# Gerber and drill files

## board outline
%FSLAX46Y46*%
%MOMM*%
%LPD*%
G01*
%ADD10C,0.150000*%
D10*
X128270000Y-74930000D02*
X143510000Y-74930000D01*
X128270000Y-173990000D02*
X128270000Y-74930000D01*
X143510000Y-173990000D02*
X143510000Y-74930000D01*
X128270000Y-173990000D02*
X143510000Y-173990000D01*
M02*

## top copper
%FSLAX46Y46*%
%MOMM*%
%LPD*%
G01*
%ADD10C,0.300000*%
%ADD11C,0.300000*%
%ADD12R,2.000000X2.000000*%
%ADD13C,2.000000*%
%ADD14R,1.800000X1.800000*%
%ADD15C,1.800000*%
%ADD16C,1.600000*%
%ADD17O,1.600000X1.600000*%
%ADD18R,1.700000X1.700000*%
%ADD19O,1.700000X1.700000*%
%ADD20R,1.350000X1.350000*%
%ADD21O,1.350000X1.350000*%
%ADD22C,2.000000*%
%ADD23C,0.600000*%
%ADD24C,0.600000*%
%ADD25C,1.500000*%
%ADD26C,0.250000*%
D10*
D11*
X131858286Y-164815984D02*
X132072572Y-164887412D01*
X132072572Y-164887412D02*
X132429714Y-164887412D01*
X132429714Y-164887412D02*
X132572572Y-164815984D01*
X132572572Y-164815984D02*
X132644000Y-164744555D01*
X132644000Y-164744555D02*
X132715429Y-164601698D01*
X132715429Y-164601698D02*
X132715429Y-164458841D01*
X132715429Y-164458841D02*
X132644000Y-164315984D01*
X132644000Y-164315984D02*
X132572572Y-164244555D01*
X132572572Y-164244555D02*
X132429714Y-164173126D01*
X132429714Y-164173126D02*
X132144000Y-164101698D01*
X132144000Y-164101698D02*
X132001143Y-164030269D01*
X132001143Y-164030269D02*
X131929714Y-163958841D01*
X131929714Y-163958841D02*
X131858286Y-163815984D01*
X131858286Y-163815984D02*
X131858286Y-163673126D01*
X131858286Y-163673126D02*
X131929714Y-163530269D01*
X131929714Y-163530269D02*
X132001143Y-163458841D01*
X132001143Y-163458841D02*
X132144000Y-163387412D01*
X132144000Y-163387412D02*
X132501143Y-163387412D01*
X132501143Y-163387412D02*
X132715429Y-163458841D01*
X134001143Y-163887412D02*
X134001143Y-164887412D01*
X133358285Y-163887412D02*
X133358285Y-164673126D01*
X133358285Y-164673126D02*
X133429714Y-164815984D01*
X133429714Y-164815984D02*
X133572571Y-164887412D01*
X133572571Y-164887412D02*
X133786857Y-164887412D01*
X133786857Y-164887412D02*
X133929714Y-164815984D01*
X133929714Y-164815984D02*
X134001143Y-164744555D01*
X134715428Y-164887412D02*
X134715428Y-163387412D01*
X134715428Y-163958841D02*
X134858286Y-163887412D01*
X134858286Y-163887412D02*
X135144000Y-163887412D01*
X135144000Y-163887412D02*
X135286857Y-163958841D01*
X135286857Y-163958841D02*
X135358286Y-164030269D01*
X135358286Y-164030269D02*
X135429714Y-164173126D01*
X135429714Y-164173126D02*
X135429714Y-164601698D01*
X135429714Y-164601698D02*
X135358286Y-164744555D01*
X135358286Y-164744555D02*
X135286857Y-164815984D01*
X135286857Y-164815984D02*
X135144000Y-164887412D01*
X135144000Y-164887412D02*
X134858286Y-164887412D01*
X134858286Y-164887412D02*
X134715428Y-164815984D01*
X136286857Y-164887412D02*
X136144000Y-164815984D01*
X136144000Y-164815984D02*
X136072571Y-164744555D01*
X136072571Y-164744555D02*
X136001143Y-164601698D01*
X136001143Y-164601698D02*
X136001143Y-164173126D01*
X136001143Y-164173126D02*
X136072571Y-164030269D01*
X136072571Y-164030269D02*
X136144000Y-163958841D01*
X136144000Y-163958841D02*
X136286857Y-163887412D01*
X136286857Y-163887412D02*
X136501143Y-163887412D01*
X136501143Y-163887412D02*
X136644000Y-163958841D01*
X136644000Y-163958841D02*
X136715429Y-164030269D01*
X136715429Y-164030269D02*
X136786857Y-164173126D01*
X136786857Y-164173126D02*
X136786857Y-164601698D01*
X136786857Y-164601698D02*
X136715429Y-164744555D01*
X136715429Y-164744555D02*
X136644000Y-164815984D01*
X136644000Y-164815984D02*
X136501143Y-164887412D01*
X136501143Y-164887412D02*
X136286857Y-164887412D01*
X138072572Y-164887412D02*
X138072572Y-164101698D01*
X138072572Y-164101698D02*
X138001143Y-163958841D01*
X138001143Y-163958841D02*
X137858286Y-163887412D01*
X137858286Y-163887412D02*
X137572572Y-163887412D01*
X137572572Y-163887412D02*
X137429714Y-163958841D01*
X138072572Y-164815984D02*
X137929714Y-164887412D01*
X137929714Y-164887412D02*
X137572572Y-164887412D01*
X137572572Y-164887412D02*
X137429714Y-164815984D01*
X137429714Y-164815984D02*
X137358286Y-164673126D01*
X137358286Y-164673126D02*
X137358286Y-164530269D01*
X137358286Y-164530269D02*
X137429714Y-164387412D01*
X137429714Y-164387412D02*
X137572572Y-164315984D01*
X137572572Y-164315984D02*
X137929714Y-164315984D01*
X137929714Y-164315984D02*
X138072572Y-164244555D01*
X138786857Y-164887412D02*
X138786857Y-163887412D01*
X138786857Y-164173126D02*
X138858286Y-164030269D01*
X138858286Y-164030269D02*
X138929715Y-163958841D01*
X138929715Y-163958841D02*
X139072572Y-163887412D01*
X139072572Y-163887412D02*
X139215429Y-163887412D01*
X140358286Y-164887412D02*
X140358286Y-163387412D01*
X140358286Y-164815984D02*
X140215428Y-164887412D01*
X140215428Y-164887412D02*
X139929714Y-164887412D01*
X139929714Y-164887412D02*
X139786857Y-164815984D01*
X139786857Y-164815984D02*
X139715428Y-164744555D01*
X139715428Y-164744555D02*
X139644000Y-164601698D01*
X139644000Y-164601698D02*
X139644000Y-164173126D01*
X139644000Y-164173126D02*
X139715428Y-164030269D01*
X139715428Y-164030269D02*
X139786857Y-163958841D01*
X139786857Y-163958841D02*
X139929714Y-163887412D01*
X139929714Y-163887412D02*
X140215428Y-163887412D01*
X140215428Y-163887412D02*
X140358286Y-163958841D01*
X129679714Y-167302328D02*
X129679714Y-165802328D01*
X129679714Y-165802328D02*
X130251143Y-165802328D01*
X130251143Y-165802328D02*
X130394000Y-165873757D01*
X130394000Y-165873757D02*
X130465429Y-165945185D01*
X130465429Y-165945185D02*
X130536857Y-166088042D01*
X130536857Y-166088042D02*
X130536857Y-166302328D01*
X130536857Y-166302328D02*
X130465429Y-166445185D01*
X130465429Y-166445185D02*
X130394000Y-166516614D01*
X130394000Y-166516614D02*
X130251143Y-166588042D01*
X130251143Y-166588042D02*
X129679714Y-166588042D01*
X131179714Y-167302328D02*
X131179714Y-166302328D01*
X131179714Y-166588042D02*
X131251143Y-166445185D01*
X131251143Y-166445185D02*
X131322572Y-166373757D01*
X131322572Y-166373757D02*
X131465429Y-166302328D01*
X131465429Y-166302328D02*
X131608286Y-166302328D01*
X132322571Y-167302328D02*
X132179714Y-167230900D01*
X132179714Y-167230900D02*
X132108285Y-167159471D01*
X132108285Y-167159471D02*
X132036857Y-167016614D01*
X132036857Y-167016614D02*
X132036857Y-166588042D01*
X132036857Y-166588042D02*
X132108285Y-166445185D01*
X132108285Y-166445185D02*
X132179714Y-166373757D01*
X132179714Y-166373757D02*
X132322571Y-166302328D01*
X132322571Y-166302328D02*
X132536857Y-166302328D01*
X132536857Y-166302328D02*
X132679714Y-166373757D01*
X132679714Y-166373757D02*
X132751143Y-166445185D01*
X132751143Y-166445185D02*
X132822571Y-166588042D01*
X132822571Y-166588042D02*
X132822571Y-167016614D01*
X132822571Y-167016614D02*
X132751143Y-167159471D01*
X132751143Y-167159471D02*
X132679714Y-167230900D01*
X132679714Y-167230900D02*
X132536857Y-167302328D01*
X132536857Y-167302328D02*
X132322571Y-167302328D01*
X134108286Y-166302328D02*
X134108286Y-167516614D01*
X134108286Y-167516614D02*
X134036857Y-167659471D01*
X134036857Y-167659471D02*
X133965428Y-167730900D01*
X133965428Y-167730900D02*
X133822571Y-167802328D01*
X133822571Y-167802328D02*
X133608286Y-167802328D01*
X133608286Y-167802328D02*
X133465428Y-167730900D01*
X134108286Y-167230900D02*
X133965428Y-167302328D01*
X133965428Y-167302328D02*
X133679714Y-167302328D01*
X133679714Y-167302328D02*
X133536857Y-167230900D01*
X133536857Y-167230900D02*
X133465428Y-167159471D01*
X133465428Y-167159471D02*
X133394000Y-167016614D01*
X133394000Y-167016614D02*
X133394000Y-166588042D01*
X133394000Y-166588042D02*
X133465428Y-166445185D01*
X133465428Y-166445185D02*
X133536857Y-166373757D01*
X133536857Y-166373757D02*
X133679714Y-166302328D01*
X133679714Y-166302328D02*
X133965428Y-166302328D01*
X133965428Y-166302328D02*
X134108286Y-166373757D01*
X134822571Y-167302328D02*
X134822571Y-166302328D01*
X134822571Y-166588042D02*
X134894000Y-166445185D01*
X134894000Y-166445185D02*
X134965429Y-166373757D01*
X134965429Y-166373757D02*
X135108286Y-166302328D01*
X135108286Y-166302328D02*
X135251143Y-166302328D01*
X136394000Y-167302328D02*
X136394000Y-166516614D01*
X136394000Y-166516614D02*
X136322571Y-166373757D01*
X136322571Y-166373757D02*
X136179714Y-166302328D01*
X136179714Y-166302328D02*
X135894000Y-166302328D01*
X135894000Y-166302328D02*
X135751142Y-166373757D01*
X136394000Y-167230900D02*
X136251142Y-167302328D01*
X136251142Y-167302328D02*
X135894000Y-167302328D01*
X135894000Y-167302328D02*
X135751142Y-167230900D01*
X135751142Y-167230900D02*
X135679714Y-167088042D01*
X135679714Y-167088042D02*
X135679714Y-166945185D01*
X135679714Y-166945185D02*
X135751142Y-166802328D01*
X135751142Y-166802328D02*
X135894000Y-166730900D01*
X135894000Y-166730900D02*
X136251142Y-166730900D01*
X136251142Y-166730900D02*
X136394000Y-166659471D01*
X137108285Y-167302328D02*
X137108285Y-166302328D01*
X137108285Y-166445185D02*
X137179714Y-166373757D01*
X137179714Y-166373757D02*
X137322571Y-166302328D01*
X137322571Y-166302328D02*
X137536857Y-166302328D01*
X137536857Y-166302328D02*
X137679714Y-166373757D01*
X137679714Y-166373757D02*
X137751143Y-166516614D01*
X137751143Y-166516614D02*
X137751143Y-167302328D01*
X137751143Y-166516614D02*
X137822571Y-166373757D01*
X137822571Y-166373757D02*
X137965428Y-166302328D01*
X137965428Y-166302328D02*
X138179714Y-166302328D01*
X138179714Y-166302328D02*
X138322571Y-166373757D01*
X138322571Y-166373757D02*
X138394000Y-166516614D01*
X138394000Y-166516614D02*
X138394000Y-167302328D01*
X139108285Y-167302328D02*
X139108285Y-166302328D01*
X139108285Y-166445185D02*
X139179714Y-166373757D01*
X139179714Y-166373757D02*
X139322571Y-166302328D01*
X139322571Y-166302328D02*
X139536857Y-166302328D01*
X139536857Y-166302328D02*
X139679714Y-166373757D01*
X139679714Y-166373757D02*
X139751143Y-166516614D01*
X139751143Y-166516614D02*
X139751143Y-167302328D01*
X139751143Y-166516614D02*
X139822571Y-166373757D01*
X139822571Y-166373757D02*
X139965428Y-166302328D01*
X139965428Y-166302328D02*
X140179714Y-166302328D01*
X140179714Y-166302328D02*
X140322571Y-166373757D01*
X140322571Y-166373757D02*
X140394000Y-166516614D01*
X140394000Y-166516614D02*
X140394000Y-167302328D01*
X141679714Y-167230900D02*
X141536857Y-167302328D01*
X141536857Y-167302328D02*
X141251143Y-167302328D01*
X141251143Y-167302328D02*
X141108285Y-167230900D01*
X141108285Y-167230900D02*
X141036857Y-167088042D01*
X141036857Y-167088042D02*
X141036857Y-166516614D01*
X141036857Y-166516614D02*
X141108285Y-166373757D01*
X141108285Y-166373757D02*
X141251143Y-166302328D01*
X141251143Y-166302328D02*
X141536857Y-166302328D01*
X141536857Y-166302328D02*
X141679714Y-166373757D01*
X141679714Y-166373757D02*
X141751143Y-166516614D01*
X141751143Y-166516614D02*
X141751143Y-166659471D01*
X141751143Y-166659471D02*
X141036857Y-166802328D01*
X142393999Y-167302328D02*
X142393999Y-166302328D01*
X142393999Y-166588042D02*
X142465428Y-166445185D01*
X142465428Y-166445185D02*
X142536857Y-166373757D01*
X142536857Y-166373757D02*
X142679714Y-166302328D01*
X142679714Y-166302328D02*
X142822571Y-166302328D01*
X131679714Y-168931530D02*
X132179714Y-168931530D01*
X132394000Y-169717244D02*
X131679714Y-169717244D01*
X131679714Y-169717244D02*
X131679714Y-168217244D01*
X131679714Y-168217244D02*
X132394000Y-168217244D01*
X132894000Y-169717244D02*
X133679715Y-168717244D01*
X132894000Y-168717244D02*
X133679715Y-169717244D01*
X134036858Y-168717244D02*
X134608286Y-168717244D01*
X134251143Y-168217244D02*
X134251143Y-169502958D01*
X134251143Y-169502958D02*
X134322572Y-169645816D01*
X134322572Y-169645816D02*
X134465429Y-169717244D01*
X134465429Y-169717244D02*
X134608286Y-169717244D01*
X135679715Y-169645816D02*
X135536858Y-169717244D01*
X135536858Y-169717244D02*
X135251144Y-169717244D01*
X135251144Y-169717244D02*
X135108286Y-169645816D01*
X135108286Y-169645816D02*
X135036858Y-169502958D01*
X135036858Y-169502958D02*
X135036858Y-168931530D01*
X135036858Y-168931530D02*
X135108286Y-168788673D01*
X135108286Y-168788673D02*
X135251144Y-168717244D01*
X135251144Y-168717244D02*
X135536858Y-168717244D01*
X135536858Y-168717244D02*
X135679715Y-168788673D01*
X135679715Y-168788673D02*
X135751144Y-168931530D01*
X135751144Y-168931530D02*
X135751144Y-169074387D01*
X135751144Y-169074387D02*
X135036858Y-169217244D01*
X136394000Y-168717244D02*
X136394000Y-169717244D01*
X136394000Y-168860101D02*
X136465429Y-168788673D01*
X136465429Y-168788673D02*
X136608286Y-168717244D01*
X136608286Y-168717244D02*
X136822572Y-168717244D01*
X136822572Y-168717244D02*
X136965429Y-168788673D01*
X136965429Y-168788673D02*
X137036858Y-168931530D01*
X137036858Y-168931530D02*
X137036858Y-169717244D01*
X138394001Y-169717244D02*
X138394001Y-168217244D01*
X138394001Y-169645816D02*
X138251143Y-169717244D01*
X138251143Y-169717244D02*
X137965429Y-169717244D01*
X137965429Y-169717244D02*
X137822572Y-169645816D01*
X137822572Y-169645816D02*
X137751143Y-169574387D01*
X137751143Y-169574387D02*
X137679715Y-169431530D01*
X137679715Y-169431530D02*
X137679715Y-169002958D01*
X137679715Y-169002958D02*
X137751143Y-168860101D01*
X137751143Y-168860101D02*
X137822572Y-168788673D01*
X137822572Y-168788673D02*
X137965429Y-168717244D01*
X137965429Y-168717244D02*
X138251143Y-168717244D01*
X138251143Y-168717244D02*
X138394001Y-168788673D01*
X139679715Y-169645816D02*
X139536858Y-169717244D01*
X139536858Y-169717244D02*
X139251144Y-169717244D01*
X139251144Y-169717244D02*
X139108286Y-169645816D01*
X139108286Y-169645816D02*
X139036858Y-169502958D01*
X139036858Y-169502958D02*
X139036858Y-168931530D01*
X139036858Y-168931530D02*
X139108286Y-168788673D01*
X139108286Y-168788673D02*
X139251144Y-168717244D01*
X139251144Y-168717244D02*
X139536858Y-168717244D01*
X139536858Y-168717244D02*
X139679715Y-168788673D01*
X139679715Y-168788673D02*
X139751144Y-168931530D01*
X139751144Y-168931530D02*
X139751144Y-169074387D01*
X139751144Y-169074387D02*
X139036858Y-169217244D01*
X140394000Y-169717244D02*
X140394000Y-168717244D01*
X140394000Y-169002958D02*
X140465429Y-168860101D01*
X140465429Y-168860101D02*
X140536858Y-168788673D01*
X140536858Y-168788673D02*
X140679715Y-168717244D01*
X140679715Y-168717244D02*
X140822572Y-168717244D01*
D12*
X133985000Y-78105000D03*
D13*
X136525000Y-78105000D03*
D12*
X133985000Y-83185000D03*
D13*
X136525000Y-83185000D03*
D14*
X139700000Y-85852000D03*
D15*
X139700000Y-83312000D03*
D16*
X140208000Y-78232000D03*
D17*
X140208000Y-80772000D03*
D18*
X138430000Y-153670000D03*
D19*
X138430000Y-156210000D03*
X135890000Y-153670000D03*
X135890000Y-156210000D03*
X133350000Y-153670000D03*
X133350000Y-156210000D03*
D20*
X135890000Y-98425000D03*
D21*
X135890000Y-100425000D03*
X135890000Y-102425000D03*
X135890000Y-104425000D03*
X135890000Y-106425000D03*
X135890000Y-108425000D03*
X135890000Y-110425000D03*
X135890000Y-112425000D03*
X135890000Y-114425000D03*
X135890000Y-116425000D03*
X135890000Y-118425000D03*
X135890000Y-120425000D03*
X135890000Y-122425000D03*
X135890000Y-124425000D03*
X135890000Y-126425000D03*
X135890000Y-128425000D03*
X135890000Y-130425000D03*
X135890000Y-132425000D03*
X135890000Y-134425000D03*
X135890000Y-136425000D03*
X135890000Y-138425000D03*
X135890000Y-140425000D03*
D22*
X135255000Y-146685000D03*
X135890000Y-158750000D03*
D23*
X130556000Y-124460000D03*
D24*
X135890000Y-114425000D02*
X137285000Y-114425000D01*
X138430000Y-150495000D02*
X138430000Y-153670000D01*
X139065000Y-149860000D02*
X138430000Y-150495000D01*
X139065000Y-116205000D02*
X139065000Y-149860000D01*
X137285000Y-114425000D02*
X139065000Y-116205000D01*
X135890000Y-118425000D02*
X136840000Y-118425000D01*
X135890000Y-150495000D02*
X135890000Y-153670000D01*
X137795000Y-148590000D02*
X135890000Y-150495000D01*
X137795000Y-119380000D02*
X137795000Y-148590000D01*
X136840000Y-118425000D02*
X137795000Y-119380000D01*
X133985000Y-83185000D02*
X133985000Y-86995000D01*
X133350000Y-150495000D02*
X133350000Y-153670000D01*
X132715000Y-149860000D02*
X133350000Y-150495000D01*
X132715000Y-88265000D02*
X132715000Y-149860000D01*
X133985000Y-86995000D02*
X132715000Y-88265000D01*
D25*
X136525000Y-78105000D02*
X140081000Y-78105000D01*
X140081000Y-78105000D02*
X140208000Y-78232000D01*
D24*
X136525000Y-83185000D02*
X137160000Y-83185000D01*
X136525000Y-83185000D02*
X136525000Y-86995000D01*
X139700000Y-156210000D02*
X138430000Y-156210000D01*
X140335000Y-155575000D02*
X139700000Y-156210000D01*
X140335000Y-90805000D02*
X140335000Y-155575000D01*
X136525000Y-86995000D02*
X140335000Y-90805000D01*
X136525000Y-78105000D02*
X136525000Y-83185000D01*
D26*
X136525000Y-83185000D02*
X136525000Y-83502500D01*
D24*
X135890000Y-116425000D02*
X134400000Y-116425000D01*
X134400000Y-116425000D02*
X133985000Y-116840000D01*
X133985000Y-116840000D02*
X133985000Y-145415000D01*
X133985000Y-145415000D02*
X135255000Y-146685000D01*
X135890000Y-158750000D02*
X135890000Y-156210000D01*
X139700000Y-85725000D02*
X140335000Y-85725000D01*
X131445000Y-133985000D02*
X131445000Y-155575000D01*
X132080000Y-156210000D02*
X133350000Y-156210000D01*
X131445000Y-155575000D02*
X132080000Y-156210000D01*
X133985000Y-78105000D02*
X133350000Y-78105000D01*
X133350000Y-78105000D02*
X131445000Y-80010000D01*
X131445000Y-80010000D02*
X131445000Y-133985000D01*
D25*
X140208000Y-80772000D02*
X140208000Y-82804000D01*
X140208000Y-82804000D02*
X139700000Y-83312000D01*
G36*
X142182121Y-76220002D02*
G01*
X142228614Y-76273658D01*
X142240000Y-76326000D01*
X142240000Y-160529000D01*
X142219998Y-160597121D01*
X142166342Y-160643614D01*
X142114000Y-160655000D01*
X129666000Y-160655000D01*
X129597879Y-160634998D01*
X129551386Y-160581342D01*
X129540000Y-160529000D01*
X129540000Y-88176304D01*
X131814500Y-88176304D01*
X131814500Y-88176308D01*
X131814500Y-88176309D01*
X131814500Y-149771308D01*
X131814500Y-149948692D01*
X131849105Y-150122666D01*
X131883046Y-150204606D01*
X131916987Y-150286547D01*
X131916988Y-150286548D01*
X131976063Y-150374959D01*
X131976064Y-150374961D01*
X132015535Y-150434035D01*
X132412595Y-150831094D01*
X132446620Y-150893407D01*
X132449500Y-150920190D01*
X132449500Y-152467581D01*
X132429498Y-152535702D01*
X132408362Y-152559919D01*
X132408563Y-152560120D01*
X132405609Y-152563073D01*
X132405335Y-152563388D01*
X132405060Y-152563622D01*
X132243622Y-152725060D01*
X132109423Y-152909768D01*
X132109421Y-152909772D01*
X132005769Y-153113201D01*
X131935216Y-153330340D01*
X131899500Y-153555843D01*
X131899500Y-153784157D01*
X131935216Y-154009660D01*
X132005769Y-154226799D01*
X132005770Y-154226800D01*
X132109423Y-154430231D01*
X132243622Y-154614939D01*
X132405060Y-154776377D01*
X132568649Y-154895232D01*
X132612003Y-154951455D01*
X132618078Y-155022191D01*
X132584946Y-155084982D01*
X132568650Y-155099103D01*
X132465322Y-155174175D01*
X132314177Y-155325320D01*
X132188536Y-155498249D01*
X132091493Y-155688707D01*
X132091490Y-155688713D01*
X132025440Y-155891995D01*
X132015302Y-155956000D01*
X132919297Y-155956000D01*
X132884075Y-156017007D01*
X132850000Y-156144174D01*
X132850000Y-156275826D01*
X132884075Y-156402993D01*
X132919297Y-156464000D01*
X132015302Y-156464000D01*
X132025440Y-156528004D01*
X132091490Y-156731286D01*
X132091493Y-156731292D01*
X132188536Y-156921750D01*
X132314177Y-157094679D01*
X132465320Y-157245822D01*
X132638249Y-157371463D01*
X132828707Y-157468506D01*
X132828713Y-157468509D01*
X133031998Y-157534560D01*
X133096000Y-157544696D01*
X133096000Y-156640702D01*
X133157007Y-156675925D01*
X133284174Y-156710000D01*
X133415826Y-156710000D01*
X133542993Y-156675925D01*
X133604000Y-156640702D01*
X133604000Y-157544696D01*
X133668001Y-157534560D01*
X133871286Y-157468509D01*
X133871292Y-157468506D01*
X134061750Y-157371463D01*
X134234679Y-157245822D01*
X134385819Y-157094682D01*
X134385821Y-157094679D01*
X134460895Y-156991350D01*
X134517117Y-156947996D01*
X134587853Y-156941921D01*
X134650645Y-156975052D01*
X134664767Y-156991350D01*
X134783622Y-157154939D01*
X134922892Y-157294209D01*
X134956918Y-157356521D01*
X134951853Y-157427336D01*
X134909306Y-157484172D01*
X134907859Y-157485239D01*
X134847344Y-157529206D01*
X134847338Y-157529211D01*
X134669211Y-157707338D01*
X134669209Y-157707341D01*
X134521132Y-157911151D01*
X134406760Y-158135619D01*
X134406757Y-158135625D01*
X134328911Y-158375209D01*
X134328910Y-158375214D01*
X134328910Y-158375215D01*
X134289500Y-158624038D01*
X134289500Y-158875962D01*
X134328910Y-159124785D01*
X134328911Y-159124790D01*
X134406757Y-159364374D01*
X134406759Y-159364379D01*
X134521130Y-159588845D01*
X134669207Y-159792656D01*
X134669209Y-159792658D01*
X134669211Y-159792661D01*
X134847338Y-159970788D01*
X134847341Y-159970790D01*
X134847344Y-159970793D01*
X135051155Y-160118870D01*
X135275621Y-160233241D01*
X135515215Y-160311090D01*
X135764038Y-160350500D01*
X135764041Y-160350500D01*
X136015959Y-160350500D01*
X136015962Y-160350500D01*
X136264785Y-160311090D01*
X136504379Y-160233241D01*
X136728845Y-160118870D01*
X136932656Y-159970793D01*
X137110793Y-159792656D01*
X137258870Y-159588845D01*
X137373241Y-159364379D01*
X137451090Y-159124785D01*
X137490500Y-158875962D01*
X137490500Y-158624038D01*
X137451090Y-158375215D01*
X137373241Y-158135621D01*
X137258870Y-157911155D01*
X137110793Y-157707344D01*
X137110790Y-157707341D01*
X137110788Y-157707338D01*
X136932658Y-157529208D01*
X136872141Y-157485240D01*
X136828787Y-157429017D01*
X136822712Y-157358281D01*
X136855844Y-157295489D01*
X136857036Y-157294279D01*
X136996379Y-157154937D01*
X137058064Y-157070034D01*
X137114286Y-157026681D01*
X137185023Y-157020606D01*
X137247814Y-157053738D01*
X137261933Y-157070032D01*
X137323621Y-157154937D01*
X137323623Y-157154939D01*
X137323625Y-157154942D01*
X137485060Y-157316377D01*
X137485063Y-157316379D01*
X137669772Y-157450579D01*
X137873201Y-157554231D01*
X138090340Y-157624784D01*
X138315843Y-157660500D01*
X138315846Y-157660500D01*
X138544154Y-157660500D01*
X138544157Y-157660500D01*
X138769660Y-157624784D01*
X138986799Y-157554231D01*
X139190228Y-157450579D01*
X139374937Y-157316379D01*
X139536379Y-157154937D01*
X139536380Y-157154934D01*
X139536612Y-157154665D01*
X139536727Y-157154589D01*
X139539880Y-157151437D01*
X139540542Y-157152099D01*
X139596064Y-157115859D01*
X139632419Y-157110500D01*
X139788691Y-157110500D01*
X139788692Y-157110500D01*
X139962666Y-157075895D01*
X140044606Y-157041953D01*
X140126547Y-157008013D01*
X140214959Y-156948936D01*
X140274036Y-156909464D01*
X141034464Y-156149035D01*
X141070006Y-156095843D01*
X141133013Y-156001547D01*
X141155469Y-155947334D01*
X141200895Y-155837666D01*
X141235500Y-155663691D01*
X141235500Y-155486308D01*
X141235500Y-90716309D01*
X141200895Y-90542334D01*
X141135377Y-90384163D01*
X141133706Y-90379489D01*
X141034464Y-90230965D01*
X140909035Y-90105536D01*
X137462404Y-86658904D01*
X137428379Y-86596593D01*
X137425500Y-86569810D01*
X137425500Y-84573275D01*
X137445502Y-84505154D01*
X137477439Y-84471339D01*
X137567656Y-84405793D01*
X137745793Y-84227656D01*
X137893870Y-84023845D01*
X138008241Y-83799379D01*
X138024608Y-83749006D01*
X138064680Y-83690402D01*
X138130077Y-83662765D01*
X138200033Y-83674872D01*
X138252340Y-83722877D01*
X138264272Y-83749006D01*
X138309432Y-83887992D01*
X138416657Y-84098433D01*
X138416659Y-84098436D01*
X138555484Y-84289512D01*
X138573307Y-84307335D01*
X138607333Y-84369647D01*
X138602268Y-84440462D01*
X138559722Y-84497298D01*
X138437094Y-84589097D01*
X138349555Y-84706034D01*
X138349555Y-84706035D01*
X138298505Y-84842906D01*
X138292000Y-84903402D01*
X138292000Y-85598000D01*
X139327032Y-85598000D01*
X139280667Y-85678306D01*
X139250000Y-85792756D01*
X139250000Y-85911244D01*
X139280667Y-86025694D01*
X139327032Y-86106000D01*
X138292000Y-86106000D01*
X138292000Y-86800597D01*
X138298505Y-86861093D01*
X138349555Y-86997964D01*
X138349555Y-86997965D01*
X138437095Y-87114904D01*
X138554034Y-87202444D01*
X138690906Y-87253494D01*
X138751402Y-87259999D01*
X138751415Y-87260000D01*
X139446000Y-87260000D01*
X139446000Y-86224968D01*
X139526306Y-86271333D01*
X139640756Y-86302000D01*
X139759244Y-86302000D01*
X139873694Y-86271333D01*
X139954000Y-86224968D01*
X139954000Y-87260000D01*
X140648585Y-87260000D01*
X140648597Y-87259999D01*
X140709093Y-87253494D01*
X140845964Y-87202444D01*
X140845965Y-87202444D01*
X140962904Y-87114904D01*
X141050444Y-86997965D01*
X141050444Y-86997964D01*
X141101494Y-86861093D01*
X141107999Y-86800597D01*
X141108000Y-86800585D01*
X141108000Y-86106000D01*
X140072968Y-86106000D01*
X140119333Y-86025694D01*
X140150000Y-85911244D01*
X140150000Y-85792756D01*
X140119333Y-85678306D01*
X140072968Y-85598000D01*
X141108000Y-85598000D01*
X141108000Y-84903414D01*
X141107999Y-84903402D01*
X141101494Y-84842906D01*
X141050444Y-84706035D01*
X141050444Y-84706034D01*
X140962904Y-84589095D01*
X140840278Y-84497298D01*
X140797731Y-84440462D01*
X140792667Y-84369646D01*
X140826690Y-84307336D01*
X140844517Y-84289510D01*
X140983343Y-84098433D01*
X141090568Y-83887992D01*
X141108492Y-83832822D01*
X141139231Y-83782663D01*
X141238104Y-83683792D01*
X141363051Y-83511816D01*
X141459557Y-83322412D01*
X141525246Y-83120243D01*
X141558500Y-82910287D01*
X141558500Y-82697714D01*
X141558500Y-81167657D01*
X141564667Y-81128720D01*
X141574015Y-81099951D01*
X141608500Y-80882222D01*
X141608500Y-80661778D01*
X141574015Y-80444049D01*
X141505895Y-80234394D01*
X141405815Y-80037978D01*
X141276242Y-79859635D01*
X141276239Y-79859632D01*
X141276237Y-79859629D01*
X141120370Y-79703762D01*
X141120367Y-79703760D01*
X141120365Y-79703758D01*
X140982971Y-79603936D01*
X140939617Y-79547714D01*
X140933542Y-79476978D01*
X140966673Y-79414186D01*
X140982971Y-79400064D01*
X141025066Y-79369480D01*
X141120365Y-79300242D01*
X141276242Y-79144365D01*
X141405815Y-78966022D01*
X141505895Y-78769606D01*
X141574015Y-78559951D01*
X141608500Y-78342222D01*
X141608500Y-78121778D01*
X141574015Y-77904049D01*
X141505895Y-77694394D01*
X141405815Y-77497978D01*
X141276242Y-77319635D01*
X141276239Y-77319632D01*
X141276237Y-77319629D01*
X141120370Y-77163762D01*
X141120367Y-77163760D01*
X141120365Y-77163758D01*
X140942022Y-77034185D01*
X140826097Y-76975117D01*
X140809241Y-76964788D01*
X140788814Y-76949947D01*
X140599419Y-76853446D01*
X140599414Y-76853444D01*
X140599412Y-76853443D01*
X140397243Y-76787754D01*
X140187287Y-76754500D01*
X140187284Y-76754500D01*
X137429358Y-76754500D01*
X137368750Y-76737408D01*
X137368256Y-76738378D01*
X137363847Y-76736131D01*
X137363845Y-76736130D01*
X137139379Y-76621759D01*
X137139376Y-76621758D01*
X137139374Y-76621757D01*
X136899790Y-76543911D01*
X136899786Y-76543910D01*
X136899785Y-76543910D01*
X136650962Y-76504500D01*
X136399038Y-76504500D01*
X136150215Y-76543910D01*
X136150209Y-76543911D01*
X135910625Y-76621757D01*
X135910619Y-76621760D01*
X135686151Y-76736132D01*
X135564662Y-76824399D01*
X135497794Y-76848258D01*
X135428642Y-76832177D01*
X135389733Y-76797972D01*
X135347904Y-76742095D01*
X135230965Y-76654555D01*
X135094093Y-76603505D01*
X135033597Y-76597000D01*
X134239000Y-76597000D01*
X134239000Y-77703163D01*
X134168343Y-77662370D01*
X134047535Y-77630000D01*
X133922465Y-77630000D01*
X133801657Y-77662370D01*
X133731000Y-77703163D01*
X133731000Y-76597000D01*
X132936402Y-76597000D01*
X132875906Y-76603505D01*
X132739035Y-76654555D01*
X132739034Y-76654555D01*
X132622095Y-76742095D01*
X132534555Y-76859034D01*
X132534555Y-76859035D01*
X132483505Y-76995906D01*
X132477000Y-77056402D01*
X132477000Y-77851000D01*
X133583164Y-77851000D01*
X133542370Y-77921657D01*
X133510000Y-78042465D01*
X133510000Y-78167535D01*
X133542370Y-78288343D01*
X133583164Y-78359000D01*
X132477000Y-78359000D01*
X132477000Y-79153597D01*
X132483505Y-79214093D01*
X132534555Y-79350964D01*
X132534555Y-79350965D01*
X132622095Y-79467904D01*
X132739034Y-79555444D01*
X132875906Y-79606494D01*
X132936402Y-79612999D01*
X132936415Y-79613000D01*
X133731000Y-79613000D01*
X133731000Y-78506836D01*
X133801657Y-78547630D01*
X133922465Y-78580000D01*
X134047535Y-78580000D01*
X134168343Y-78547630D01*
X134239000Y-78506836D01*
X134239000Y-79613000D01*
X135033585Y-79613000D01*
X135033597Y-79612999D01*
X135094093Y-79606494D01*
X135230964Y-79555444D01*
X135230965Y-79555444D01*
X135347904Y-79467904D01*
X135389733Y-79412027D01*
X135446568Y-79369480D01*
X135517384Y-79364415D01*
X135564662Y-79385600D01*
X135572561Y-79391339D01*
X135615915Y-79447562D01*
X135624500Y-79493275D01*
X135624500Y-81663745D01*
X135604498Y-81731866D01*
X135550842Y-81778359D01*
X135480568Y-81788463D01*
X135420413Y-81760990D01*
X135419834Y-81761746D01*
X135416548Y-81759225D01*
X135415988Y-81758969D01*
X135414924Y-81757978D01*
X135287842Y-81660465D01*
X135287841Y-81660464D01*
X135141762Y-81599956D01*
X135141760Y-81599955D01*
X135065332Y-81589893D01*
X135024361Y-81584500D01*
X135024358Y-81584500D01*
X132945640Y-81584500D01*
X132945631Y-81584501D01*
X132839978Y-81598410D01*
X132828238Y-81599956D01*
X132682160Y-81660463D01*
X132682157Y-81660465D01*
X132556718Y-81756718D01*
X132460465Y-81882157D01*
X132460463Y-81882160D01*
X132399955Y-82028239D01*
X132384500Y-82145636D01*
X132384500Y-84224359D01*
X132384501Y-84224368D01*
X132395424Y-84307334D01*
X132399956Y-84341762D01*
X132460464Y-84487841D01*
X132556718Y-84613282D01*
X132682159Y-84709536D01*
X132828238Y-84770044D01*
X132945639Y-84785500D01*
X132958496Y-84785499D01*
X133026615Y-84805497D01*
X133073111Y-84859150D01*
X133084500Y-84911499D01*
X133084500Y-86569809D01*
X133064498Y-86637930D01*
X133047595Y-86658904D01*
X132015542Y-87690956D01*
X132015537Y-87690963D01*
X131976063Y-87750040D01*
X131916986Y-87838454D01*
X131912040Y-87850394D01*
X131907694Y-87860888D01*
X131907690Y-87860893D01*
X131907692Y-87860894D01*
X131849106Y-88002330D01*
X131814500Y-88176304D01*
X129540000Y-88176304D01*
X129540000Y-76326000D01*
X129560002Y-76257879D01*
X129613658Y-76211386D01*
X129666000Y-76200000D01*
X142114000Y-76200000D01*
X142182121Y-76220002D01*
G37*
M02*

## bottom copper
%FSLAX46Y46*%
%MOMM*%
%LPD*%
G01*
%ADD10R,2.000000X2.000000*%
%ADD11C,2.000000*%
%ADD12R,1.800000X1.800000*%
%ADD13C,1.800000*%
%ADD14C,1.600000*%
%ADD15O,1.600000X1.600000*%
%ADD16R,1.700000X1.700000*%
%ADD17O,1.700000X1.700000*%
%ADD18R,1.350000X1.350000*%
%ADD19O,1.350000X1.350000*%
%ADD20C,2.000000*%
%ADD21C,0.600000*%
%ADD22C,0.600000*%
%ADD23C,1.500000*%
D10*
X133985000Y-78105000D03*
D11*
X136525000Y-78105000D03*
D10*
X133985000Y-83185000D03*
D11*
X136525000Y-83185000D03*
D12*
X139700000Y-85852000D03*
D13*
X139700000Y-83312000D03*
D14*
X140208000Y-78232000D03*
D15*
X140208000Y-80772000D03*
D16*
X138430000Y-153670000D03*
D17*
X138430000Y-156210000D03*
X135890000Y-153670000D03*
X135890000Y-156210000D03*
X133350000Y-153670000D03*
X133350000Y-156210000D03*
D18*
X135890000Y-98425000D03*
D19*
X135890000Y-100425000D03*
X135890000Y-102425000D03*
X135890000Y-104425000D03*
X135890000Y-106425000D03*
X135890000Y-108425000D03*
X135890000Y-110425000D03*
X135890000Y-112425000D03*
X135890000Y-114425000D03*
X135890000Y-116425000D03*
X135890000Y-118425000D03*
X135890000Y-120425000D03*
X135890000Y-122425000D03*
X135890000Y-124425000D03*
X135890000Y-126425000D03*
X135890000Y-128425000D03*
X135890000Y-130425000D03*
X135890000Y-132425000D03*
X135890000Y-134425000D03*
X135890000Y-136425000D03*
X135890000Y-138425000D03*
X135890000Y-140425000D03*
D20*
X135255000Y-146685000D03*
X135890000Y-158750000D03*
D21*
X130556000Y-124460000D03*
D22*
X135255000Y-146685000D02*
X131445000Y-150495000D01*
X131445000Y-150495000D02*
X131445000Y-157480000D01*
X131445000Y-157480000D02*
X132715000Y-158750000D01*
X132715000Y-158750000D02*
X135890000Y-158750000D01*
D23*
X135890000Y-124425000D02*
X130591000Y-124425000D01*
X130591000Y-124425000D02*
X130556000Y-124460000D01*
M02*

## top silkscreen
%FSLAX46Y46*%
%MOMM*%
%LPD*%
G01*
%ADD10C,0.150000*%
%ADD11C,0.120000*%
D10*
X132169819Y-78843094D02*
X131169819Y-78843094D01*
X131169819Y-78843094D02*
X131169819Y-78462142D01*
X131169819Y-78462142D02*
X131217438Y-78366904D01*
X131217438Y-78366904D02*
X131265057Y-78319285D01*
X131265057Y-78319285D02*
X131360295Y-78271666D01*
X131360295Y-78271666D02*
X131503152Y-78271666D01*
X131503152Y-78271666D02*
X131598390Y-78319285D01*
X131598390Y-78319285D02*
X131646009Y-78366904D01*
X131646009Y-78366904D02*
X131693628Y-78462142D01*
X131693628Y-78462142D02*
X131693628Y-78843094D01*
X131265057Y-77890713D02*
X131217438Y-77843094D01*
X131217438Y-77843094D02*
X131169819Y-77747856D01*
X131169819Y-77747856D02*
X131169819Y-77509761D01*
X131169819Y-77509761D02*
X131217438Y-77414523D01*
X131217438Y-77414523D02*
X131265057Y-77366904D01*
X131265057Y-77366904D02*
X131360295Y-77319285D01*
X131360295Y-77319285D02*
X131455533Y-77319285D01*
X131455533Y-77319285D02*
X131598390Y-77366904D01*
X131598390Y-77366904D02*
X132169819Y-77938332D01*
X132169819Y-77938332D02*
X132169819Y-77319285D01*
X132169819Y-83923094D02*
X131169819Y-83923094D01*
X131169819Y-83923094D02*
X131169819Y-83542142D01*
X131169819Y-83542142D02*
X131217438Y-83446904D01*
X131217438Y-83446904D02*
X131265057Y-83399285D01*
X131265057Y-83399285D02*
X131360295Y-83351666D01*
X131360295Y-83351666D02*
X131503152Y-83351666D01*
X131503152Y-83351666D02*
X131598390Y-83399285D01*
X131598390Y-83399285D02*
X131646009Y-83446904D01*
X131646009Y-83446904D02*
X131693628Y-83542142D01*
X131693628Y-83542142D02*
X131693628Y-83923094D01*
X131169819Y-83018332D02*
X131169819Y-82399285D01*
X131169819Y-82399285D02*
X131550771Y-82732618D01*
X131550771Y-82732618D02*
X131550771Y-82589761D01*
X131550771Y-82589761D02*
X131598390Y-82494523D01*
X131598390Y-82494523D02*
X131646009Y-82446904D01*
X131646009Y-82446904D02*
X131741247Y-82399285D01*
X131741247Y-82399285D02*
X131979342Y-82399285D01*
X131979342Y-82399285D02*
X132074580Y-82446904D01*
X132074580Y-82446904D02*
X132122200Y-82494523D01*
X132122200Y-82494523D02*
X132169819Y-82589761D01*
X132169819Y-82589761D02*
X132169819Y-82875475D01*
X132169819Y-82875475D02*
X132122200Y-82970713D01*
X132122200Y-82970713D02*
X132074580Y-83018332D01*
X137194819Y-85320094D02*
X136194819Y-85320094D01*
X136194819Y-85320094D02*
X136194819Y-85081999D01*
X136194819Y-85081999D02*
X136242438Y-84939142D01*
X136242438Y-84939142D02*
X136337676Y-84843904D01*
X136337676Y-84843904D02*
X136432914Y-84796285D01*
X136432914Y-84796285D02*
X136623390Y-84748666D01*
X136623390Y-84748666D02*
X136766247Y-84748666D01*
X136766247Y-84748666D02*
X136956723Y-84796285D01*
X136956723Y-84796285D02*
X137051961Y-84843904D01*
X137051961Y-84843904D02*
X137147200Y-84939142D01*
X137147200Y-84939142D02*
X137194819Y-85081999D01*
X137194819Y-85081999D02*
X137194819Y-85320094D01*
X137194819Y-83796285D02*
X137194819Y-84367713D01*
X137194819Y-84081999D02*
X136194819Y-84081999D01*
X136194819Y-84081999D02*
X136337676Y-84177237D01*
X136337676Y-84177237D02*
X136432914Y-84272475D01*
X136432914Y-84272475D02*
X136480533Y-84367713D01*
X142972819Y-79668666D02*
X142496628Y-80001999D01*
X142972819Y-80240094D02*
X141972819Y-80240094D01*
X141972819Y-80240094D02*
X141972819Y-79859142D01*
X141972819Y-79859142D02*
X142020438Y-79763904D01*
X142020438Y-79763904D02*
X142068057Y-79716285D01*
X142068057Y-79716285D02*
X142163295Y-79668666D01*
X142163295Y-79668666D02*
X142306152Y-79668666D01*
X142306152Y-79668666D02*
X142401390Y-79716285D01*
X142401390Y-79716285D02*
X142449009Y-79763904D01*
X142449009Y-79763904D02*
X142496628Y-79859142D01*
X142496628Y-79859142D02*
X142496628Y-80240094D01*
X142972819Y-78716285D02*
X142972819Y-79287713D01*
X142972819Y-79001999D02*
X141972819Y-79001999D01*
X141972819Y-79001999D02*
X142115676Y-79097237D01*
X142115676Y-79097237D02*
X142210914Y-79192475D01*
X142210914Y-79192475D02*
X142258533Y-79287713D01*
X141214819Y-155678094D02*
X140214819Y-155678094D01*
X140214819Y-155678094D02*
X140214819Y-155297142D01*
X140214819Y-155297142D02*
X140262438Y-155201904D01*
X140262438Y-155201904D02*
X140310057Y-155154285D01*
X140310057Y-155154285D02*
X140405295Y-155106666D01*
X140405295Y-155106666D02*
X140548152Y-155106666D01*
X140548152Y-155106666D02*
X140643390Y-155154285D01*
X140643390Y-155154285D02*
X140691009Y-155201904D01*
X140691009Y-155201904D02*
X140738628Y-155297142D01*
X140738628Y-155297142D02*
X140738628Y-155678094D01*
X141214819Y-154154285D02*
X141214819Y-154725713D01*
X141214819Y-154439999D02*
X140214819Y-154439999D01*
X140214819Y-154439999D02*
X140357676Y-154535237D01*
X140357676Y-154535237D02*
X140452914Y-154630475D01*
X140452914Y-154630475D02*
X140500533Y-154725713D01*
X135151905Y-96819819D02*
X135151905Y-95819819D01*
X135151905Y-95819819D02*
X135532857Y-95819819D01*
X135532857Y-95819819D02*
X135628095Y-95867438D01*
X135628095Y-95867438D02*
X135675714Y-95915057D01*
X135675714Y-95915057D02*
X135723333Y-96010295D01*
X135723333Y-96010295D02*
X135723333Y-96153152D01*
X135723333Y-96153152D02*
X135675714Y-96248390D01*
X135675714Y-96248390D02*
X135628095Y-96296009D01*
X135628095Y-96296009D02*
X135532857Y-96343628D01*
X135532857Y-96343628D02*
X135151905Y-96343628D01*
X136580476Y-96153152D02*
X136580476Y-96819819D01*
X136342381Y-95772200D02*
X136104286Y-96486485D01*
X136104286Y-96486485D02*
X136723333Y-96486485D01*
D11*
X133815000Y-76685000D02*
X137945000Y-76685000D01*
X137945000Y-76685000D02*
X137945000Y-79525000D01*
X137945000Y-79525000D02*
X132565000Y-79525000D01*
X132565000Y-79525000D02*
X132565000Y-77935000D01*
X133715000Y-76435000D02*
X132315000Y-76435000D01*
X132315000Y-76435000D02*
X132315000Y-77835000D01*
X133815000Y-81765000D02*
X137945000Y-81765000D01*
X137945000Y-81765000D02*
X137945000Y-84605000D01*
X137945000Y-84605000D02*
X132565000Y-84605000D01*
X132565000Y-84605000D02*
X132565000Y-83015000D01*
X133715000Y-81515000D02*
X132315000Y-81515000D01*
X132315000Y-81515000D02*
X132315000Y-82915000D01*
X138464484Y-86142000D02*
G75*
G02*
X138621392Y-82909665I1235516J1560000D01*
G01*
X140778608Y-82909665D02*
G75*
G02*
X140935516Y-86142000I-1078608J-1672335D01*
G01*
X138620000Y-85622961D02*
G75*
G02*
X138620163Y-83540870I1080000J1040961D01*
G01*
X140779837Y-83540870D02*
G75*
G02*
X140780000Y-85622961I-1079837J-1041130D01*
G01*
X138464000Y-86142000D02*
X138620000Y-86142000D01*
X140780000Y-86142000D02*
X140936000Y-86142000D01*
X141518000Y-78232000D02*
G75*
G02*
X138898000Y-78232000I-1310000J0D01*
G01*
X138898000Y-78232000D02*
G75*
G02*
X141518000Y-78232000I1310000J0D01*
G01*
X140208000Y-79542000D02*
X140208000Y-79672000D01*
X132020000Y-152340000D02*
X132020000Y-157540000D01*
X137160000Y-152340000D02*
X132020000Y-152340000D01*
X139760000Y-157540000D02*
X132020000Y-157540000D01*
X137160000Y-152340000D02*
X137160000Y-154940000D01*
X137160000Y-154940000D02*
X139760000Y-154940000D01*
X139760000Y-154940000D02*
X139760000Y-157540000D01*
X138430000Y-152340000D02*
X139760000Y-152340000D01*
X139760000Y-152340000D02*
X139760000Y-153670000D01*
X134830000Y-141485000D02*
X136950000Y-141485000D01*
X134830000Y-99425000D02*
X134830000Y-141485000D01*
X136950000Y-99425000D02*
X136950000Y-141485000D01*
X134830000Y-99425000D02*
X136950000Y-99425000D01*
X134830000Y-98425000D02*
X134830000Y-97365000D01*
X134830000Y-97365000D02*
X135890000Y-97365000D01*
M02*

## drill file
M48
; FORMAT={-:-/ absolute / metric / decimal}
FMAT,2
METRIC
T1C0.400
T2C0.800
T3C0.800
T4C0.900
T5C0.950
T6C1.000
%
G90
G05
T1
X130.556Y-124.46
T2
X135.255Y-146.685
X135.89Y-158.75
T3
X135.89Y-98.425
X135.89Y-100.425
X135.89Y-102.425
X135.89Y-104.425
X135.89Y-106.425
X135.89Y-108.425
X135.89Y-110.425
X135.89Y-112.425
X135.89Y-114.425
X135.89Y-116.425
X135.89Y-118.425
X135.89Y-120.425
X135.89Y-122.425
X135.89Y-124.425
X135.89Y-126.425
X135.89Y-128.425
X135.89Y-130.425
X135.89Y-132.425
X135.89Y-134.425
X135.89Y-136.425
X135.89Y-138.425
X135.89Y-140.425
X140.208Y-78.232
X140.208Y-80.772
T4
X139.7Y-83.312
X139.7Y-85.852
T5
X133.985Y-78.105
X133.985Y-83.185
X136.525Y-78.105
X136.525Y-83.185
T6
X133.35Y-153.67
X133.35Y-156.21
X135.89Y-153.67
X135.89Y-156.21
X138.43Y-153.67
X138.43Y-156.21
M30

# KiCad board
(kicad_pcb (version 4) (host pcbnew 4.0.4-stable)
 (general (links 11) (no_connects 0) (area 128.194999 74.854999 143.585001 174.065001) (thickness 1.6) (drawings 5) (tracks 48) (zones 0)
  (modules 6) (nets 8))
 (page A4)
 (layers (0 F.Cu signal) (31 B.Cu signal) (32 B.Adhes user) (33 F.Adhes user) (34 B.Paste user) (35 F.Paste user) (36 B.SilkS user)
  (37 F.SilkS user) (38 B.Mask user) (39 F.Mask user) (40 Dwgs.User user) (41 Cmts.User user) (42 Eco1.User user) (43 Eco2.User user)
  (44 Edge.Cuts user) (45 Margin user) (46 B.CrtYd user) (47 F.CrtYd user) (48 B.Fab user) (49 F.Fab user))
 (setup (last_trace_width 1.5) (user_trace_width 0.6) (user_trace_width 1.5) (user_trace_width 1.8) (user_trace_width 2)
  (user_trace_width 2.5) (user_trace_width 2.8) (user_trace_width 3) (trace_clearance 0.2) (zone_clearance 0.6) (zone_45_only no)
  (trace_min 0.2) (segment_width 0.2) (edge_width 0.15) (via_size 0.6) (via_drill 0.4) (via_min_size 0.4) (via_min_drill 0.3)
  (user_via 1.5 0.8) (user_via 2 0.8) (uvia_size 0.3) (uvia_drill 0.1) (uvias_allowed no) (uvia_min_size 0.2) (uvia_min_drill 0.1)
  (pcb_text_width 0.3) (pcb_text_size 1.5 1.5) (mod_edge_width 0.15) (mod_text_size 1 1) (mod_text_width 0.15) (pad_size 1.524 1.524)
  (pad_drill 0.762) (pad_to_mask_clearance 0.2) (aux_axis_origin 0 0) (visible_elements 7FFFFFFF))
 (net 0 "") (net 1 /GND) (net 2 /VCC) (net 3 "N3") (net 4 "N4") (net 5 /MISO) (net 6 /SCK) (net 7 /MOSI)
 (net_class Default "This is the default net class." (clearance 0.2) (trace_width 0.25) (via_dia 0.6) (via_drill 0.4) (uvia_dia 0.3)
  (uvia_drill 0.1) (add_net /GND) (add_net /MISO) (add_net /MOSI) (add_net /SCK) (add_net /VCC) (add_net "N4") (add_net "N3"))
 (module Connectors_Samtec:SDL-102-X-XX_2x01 (layer F.Cu) (at 133.985 78.105)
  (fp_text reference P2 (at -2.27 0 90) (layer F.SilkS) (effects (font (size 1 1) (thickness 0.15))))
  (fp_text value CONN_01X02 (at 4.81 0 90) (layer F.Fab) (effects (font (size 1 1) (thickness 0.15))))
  (fp_line (start -0.17 -1.42) (end 3.96 -1.42) (layer F.SilkS) (width 0.12))
  (fp_line (start 3.96 -1.42) (end 3.96 1.42) (layer F.SilkS) (width 0.12))
  (fp_line (start 3.96 1.42) (end -1.42 1.42) (layer F.SilkS) (width 0.12))
  (fp_line (start -1.42 1.42) (end -1.42 -0.17) (layer F.SilkS) (width 0.12))
  (fp_line (start -0.27 -1.67) (end -1.67 -1.67) (layer F.SilkS) (width 0.12))
  (fp_line (start -1.67 -1.67) (end -1.67 -0.27) (layer F.SilkS) (width 0.12))
  (pad 1 thru_hole rect (at 0 0) (size 2 2) (drill 0.95) (layers *.Cu *.Mask) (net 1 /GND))
  (pad 2 thru_hole circle (at 2.54 0) (size 2 2) (drill 0.95) (layers *.Cu *.Mask) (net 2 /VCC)))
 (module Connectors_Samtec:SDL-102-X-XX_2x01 (layer F.Cu) (at 133.985 83.185)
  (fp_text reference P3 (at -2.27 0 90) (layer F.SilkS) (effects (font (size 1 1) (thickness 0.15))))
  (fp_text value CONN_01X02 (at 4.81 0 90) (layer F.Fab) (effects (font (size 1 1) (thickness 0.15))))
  (fp_line (start -0.17 -1.42) (end 3.96 -1.42) (layer F.SilkS) (width 0.12))
  (fp_line (start 3.96 -1.42) (end 3.96 1.42) (layer F.SilkS) (width 0.12))
  (fp_line (start 3.96 1.42) (end -1.42 1.42) (layer F.SilkS) (width 0.12))
  (fp_line (start -1.42 1.42) (end -1.42 -0.17) (layer F.SilkS) (width 0.12))
  (fp_line (start -0.27 -1.67) (end -1.67 -1.67) (layer F.SilkS) (width 0.12))
  (fp_line (start -1.67 -1.67) (end -1.67 -0.27) (layer F.SilkS) (width 0.12))
  (pad 1 thru_hole rect (at 0 0) (size 2 2) (drill 0.95) (layers *.Cu *.Mask) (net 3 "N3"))
  (pad 2 thru_hole circle (at 2.54 0) (size 2 2) (drill 0.95) (layers *.Cu *.Mask) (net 2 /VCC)))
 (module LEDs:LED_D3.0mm (layer F.Cu) (at 139.7 85.852 90)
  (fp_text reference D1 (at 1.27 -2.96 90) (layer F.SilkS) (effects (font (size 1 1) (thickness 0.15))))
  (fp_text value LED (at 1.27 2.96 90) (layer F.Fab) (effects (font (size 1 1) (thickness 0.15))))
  (fp_arc (start 1.27 0) (end -0.29 -1.235516) (angle 108.8) (layer F.SilkS) (width 0.12))
  (fp_arc (start 1.27 0) (end -0.29 1.235516) (angle -108.8) (layer F.SilkS) (width 0.12))
  (fp_arc (start 1.27 0) (end 0.229039 -1.08) (angle 87.9) (layer F.SilkS) (width 0.12))
  (fp_arc (start 1.27 0) (end 0.229039 1.08) (angle -87.9) (layer F.SilkS) (width 0.12))
  (fp_line (start -0.29 -1.236) (end -0.29 -1.08) (layer F.SilkS) (width 0.12))
  (fp_line (start -0.29 1.08) (end -0.29 1.236) (layer F.SilkS) (width 0.12))
  (pad 1 thru_hole rect (at 0 0 90) (size 1.8 1.8) (drill 0.9) (layers *.Cu *.Mask) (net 1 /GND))
  (pad 2 thru_hole circle (at 2.54 0 90) (size 1.8 1.8) (drill 0.9) (layers *.Cu *.Mask) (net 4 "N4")))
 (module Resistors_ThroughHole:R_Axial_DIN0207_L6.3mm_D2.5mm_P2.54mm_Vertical (layer F.Cu) (at 140.208 78.232 270)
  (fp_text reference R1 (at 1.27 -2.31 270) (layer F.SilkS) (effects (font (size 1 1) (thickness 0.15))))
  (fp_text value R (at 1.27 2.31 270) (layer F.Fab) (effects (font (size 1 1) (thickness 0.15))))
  (fp_circle (center 0 0) (end 1.31 0) (layer F.SilkS) (width 0.12))
  (fp_line (start 1.31 0) (end 1.44 0) (layer F.SilkS) (width 0.12))
  (pad 1 thru_hole circle (at 0 0 270) (size 1.6 1.6) (drill 0.8) (layers *.Cu *.Mask) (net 2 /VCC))
  (pad 2 thru_hole oval (at 2.54 0 270) (size 1.6 1.6) (drill 0.8) (layers *.Cu *.Mask) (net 4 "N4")))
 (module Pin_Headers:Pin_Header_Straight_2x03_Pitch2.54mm (layer F.Cu) (at 138.43 153.67 270)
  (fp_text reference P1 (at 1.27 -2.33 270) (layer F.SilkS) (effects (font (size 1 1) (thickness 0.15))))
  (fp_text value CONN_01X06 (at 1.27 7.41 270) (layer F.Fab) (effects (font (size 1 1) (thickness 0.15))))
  (fp_line (start -1.33 6.41) (end 3.87 6.41) (layer F.SilkS) (width 0.12))
  (fp_line (start -1.33 1.27) (end -1.33 6.41) (layer F.SilkS) (width 0.12))
  (fp_line (start 3.87 -1.33) (end 3.87 6.41) (layer F.SilkS) (width 0.12))
  (fp_line (start -1.33 1.27) (end 1.27 1.27) (layer F.SilkS) (width 0.12))
  (fp_line (start 1.27 1.27) (end 1.27 -1.33) (layer F.SilkS) (width 0.12))
  (fp_line (start 1.27 -1.33) (end 3.87 -1.33) (layer F.SilkS) (width 0.12))
  (fp_line (start -1.33 0) (end -1.33 -1.33) (layer F.SilkS) (width 0.12))
  (fp_line (start -1.33 -1.33) (end 0 -1.33) (layer F.SilkS) (width 0.12))
  (pad 1 thru_hole rect (at 0 0 270) (size 1.7 1.7) (drill 1) (layers *.Cu *.Mask) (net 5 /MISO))
  (pad 2 thru_hole oval (at 2.54 0 270) (size 1.7 1.7) (drill 1) (layers *.Cu *.Mask) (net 2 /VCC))
  (pad 3 thru_hole oval (at 0 2.54 270) (size 1.7 1.7) (drill 1) (layers *.Cu *.Mask) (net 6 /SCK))
  (pad 4 thru_hole oval (at 2.54 2.54 270) (size 1.7 1.7) (drill 1) (layers *.Cu *.Mask) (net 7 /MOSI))
  (pad 5 thru_hole oval (at 0 5.08 270) (size 1.7 1.7) (drill 1) (layers *.Cu *.Mask) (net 3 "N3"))
  (pad 6 thru_hole oval (at 2.54 5.08 270) (size 1.7 1.7) (drill 1) (layers *.Cu *.Mask) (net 1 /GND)))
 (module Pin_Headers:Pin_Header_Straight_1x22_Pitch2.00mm (layer F.Cu) (at 135.89 98.425)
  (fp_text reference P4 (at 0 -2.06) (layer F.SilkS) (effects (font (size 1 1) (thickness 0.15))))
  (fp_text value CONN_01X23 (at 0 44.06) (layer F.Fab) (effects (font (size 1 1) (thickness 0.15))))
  (fp_line (start -1.06 43.06) (end 1.06 43.06) (layer F.SilkS) (width 0.12))
  (fp_line (start -1.06 1) (end -1.06 43.06) (layer F.SilkS) (width 0.12))
  (fp_line (start 1.06 1) (end 1.06 43.06) (layer F.SilkS) (width 0.12))
  (fp_line (start -1.06 1) (end 1.06 1) (layer F.SilkS) (width 0.12))
  (fp_line (start -1.06 0) (end -1.06 -1.06) (layer F.SilkS) (width 0.12))
  (fp_line (start -1.06 -1.06) (end 0 -1.06) (layer F.SilkS) (width 0.12))
  (pad 1 thru_hole rect (at 0 0) (size 1.35 1.35) (drill 0.8) (layers *.Cu *.Mask))
  (pad 2 thru_hole oval (at 0 2) (size 1.35 1.35) (drill 0.8) (layers *.Cu *.Mask))
  (pad 3 thru_hole oval (at 0 4) (size 1.35 1.35) (drill 0.8) (layers *.Cu *.Mask))
  (pad 4 thru_hole oval (at 0 6) (size 1.35 1.35) (drill 0.8) (layers *.Cu *.Mask))
  (pad 5 thru_hole oval (at 0 8) (size 1.35 1.35) (drill 0.8) (layers *.Cu *.Mask))
  (pad 6 thru_hole oval (at 0 10) (size 1.35 1.35) (drill 0.8) (layers *.Cu *.Mask))
  (pad 7 thru_hole oval (at 0 12) (size 1.35 1.35) (drill 0.8) (layers *.Cu *.Mask))
  (pad 8 thru_hole oval (at 0 14) (size 1.35 1.35) (drill 0.8) (layers *.Cu *.Mask))
  (pad 9 thru_hole oval (at 0 16) (size 1.35 1.35) (drill 0.8) (layers *.Cu *.Mask) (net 5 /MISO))
  (pad 10 thru_hole oval (at 0 18) (size 1.35 1.35) (drill 0.8) (layers *.Cu *.Mask) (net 7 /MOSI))
  (pad 11 thru_hole oval (at 0 20) (size 1.35 1.35) (drill 0.8) (layers *.Cu *.Mask) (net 6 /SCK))
  (pad 12 thru_hole oval (at 0 22) (size 1.35 1.35) (drill 0.8) (layers *.Cu *.Mask))
  (pad 13 thru_hole oval (at 0 24) (size 1.35 1.35) (drill 0.8) (layers *.Cu *.Mask))
  (pad 14 thru_hole oval (at 0 26) (size 1.35 1.35) (drill 0.8) (layers *.Cu *.Mask) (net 1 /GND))
  (pad 15 thru_hole oval (at 0 28) (size 1.35 1.35) (drill 0.8) (layers *.Cu *.Mask))
  (pad 16 thru_hole oval (at 0 30) (size 1.35 1.35) (drill 0.8) (layers *.Cu *.Mask))
  (pad 17 thru_hole oval (at 0 32) (size 1.35 1.35) (drill 0.8) (layers *.Cu *.Mask))
  (pad 18 thru_hole oval (at 0 34) (size 1.35 1.35) (drill 0.8) (layers *.Cu *.Mask))
  (pad 19 thru_hole oval (at 0 36) (size 1.35 1.35) (drill 0.8) (layers *.Cu *.Mask))
  (pad 20 thru_hole oval (at 0 38) (size 1.35 1.35) (drill 0.8) (layers *.Cu *.Mask))
  (pad 21 thru_hole oval (at 0 40) (size 1.35 1.35) (drill 0.8) (layers *.Cu *.Mask))
  (pad 22 thru_hole oval (at 0 42) (size 1.35 1.35) (drill 0.8) (layers *.Cu *.Mask)))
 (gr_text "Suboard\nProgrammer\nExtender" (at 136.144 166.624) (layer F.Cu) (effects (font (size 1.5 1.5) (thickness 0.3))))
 (gr_line (start 128.27 74.93) (end 143.51 74.93) (angle 90) (layer Edge.Cuts) (width 0.15))
 (gr_line (start 128.27 173.99) (end 128.27 74.93) (angle 90) (layer Edge.Cuts) (width 0.15))
 (gr_line (start 143.51 173.99) (end 143.51 74.93) (angle 90) (layer Edge.Cuts) (width 0.15))
 (gr_line (start 128.27 173.99) (end 143.51 173.99) (angle 90) (layer Edge.Cuts) (width 0.15))
 (segment (start 135.89 114.425) (end 137.285 114.425) (width 0.6) (layer F.Cu) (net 5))
 (segment (start 138.43 150.495) (end 138.43 153.67) (width 0.6) (layer F.Cu) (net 5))
 (segment (start 139.065 149.86) (end 138.43 150.495) (width 0.6) (layer F.Cu) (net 5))
 (segment (start 139.065 116.205) (end 139.065 149.86) (width 0.6) (layer F.Cu) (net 5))
 (segment (start 137.285 114.425) (end 139.065 116.205) (width 0.6) (layer F.Cu) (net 5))
 (segment (start 135.89 118.425) (end 136.84 118.425) (width 0.6) (layer F.Cu) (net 6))
 (segment (start 135.89 150.495) (end 135.89 153.67) (width 0.6) (layer F.Cu) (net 6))
 (segment (start 137.795 148.59) (end 135.89 150.495) (width 0.6) (layer F.Cu) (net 6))
 (segment (start 137.795 119.38) (end 137.795 148.59) (width 0.6) (layer F.Cu) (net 6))
 (segment (start 136.84 118.425) (end 137.795 119.38) (width 0.6) (layer F.Cu) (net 6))
 (segment (start 133.985 83.185) (end 133.985 86.995) (width 0.6) (layer F.Cu) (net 3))
 (segment (start 133.35 150.495) (end 133.35 153.67) (width 0.6) (layer F.Cu) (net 3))
 (segment (start 132.715 149.86) (end 133.35 150.495) (width 0.6) (layer F.Cu) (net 3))
 (segment (start 132.715 88.265) (end 132.715 149.86) (width 0.6) (layer F.Cu) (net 3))
 (segment (start 133.985 86.995) (end 132.715 88.265) (width 0.6) (layer F.Cu) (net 3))
 (segment (start 136.525 78.105) (end 140.081 78.105) (width 1.5) (layer F.Cu) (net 2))
 (segment (start 140.081 78.105) (end 140.208 78.232) (width 1.5) (layer F.Cu) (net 2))
 (segment (start 136.525 83.185) (end 137.16 83.185) (width 0.6) (layer F.Cu) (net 2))
 (segment (start 136.525 83.185) (end 136.525 86.995) (width 0.6) (layer F.Cu) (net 2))
 (segment (start 139.7 156.21) (end 138.43 156.21) (width 0.6) (layer F.Cu) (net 2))
 (segment (start 140.335 155.575) (end 139.7 156.21) (width 0.6) (layer F.Cu) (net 2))
 (segment (start 140.335 90.805) (end 140.335 155.575) (width 0.6) (layer F.Cu) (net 2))
 (segment (start 136.525 86.995) (end 140.335 90.805) (width 0.6) (layer F.Cu) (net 2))
 (segment (start 136.525 78.105) (end 136.525 83.185) (width 0.6) (layer F.Cu) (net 2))
 (segment (start 136.525 83.185) (end 136.525 83.5025) (width 0.25) (layer F.Cu) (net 2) (status 30))
 (segment (start 135.89 116.425) (end 134.4 116.425) (width 0.6) (layer F.Cu) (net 7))
 (segment (start 134.4 116.425) (end 133.985 116.84) (width 0.6) (layer F.Cu) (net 7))
 (segment (start 133.985 116.84) (end 133.985 145.415) (width 0.6) (layer F.Cu) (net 7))
 (segment (start 133.985 145.415) (end 135.255 146.685) (width 0.6) (layer F.Cu) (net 7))
 (via (at 135.255 146.685) (size 2) (drill 0.8) (layers F.Cu B.Cu) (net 7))
 (segment (start 135.255 146.685) (end 131.445 150.495) (width 0.6) (layer B.Cu) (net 7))
 (segment (start 131.445 150.495) (end 131.445 157.48) (width 0.6) (layer B.Cu) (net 7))
 (segment (start 131.445 157.48) (end 132.715 158.75) (width 0.6) (layer B.Cu) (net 7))
 (segment (start 132.715 158.75) (end 135.89 158.75) (width 0.6) (layer B.Cu) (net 7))
 (via (at 135.89 158.75) (size 2) (drill 0.8) (layers F.Cu B.Cu) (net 7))
 (segment (start 135.89 158.75) (end 135.89 156.21) (width 0.6) (layer F.Cu) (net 7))
 (segment (start 135.89 124.425) (end 130.591 124.425) (width 1.5) (layer B.Cu) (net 1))
 (via (at 130.556 124.46) (size 0.6) (drill 0.4) (layers F.Cu B.Cu) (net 1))
 (segment (start 130.591 124.425) (end 130.556 124.46) (width 1.5) (layer B.Cu) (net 1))
 (segment (start 139.7 85.725) (end 140.335 85.725) (width 0.6) (layer F.Cu) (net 1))
 (segment (start 131.445 133.985) (end 131.445 155.575) (width 0.6) (layer F.Cu) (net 1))
 (segment (start 132.08 156.21) (end 133.35 156.21) (width 0.6) (layer F.Cu) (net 1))
 (segment (start 131.445 155.575) (end 132.08 156.21) (width 0.6) (layer F.Cu) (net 1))
 (segment (start 133.985 78.105) (end 133.35 78.105) (width 0.6) (layer F.Cu) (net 1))
 (segment (start 133.35 78.105) (end 131.445 80.01) (width 0.6) (layer F.Cu) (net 1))
 (segment (start 131.445 80.01) (end 131.445 133.985) (width 0.6) (layer F.Cu) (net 1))
 (segment (start 140.208 80.772) (end 140.208 82.804) (width 1.5) (layer F.Cu) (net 4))
 (segment (start 140.208 82.804) (end 139.7 83.312) (width 1.5) (layer F.Cu) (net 4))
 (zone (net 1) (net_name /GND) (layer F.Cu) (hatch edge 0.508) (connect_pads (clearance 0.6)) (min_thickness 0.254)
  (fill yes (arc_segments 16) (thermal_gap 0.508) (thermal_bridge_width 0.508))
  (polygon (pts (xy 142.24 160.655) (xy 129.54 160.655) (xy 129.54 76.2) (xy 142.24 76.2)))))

